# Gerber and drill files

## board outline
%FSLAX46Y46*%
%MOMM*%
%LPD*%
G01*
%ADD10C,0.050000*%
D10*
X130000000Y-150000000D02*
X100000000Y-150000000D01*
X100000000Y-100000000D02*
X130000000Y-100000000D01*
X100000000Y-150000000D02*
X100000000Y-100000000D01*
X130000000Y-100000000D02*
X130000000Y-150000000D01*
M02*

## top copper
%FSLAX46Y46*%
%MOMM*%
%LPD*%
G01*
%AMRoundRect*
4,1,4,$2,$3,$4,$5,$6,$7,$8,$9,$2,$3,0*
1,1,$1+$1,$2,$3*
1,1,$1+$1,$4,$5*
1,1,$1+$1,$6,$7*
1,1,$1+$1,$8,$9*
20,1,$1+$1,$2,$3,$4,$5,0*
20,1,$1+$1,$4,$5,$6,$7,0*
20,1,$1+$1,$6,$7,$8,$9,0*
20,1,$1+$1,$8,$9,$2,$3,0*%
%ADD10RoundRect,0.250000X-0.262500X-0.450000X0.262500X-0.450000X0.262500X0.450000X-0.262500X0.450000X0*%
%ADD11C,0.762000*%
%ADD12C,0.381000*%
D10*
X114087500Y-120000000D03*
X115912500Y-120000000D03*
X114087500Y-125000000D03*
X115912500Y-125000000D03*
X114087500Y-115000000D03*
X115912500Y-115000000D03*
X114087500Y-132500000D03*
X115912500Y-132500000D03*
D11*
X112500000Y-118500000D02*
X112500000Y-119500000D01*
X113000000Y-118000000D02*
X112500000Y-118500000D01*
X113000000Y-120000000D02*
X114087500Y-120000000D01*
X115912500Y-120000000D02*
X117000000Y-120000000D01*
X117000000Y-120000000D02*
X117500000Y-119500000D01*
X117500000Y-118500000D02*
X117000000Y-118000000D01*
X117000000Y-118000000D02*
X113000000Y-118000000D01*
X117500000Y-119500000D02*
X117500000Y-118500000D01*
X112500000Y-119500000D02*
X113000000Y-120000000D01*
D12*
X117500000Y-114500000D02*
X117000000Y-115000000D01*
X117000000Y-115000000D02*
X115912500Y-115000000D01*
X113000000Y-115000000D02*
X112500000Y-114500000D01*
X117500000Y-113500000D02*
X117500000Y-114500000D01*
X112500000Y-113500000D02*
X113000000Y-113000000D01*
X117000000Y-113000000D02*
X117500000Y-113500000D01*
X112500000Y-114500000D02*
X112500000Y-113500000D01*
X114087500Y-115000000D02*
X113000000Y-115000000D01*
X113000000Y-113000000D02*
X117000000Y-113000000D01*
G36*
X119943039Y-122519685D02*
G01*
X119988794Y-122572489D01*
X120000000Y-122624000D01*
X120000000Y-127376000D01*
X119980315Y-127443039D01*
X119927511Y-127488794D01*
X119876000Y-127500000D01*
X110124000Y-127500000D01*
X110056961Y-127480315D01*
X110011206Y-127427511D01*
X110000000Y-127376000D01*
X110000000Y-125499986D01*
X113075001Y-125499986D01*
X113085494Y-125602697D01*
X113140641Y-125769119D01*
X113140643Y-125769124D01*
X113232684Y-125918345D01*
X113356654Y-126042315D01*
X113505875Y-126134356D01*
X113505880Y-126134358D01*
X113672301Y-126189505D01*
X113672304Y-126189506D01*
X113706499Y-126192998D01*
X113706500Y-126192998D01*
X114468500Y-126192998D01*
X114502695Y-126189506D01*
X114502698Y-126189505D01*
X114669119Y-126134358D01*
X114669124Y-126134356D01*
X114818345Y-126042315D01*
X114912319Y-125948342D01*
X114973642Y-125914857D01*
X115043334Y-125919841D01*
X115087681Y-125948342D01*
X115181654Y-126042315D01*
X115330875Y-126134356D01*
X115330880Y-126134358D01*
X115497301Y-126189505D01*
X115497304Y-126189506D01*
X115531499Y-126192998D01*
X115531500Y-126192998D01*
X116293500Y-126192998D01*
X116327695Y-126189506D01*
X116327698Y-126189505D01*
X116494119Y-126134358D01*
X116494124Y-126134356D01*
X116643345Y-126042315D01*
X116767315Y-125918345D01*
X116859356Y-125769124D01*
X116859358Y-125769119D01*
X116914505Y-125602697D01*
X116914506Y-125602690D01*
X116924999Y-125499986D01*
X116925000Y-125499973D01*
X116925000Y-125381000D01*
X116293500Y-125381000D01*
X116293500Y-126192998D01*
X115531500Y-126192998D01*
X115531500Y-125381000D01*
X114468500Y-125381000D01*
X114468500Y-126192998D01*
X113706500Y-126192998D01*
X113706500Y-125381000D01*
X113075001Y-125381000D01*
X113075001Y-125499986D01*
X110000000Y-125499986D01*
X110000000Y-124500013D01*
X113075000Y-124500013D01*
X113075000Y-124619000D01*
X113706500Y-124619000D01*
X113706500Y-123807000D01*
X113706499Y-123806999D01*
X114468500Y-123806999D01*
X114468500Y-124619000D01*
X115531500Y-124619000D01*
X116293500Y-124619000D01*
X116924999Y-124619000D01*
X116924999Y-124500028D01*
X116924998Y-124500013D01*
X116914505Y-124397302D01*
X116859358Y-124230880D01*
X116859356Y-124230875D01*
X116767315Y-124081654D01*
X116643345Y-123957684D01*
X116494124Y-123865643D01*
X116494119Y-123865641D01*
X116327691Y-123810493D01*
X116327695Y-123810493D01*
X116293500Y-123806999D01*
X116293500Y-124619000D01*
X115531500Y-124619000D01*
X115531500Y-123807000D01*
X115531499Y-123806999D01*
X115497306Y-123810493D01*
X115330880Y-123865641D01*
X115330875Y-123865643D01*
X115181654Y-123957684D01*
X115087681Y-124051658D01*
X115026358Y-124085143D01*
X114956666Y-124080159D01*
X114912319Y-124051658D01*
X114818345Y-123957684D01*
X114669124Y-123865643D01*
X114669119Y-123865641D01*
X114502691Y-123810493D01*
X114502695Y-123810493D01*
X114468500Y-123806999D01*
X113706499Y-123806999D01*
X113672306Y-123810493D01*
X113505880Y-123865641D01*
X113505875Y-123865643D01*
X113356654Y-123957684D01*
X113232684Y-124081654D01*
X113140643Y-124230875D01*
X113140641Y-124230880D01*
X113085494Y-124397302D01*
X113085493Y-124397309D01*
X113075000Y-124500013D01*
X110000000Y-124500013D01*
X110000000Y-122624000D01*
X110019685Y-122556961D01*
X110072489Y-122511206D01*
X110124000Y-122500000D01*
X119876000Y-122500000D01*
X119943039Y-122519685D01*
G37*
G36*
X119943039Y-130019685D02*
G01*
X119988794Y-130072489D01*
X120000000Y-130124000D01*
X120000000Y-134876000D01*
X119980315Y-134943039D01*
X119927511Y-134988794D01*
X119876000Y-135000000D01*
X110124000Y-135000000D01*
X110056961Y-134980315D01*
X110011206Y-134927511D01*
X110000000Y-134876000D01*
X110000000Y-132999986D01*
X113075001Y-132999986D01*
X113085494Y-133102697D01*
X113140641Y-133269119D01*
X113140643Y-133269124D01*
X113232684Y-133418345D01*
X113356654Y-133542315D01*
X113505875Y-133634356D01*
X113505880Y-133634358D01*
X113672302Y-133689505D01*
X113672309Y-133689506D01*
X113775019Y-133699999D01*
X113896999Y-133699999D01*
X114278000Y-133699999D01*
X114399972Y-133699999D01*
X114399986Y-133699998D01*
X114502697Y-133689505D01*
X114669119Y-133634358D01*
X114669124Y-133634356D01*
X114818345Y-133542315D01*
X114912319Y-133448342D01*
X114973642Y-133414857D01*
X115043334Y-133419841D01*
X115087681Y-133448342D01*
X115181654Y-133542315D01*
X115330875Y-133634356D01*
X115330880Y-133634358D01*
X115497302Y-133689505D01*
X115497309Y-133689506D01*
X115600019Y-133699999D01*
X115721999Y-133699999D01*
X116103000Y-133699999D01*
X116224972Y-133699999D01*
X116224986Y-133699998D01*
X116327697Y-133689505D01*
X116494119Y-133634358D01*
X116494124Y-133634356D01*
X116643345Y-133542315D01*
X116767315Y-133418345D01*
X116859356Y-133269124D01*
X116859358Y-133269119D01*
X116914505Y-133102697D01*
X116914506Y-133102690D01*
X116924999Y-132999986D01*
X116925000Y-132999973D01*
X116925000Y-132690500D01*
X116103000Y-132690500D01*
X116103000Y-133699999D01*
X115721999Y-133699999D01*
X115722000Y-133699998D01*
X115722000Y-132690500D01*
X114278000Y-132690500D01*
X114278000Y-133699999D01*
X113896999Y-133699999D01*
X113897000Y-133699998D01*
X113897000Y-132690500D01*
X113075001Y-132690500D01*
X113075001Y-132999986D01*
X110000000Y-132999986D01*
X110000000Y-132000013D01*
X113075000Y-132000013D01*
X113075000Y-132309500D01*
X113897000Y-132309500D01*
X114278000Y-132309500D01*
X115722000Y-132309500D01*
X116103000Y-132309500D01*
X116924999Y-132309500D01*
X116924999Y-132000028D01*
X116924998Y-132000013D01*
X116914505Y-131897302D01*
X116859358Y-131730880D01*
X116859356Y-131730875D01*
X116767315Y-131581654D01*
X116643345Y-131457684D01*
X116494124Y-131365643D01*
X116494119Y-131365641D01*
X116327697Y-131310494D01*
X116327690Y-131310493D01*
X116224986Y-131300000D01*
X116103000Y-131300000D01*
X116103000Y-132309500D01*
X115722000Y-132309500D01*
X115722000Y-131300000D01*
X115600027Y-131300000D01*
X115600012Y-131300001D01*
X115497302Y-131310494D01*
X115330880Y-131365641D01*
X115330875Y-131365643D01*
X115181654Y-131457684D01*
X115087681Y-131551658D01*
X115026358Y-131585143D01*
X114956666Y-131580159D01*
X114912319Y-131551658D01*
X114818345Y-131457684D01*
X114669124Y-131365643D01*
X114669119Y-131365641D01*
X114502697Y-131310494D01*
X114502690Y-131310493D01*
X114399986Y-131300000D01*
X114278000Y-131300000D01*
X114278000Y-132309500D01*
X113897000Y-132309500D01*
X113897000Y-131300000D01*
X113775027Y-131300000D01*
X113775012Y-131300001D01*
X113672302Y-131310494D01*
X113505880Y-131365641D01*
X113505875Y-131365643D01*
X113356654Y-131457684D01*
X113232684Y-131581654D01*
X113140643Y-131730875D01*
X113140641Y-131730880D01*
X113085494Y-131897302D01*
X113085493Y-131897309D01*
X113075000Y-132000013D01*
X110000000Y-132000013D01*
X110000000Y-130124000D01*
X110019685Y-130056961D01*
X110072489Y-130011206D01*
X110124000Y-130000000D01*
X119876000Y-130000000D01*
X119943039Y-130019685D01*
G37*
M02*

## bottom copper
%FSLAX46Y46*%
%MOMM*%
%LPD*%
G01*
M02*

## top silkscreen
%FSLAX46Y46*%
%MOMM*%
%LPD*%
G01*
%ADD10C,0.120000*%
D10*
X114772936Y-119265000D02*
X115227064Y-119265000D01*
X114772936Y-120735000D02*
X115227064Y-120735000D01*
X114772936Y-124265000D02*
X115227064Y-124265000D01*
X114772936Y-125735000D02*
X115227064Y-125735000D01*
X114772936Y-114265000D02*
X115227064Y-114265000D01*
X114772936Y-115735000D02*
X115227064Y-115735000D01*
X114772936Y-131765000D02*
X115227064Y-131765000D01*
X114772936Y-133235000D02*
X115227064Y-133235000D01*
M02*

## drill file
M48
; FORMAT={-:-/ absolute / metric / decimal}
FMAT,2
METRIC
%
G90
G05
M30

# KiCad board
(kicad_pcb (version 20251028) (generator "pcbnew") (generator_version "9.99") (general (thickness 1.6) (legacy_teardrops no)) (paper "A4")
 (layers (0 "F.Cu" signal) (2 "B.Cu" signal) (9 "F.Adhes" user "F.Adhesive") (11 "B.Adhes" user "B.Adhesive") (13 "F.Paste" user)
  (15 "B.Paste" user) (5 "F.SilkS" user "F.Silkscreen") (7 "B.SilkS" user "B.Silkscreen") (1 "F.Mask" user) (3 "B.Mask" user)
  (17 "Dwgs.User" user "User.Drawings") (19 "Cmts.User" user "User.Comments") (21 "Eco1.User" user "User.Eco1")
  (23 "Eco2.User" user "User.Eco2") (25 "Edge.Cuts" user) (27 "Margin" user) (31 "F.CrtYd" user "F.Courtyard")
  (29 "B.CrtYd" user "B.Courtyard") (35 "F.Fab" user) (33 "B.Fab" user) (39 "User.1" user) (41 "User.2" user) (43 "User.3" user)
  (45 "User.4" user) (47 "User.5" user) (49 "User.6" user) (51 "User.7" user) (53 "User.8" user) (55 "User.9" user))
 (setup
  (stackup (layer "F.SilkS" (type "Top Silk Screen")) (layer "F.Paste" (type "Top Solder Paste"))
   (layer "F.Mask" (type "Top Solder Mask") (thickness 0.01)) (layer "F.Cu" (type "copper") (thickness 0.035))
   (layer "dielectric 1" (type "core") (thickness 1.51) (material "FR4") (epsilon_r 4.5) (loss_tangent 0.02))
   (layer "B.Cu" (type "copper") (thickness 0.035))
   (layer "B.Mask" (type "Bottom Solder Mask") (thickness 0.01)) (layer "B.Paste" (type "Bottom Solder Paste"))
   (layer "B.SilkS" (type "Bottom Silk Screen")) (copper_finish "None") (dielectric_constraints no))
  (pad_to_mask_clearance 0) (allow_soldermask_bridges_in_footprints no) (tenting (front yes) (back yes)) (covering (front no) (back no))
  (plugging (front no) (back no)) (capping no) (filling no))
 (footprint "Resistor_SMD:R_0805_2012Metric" (layer "F.Cu") (at 115 120)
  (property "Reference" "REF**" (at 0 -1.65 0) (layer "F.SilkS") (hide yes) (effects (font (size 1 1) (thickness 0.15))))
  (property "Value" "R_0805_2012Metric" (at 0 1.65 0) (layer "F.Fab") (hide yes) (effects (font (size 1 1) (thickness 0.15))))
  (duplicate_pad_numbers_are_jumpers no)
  (fp_line (start -0.227064 -0.735) (end 0.227064 -0.735) (stroke (width 0.12) (type solid)) (layer "F.SilkS"))
  (fp_line (start -0.227064 0.735) (end 0.227064 0.735) (stroke (width 0.12) (type solid)) (layer "F.SilkS"))
  (pad "1" smd roundrect (at -0.9125 0) (size 1.025 1.4) (layers "F.Cu" "F.Mask" "F.Paste") (roundrect_rratio 0.243902) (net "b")
   (tenting (front none) (back none)))
  (pad "2" smd roundrect (at 0.9125 0) (size 1.025 1.4) (layers "F.Cu" "F.Mask" "F.Paste") (roundrect_rratio 0.243902) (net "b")
   (tenting (front none) (back none))))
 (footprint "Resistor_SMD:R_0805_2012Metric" (layer "F.Cu") (at 115 125)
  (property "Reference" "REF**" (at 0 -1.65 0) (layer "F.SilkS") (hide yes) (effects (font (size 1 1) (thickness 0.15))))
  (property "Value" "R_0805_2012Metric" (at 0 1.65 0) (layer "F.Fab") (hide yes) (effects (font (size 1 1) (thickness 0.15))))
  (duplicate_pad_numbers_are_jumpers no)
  (fp_line (start -0.227064 -0.735) (end 0.227064 -0.735) (stroke (width 0.12) (type solid)) (layer "F.SilkS"))
  (fp_line (start -0.227064 0.735) (end 0.227064 0.735) (stroke (width 0.12) (type solid)) (layer "F.SilkS"))
  (pad "1" smd roundrect (at -0.9125 0) (size 1.025 1.4) (layers "F.Cu" "F.Mask" "F.Paste") (roundrect_rratio 0.243902) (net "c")
   (tenting (front none) (back none)))
  (pad "2" smd roundrect (at 0.9125 0) (size 1.025 1.4) (layers "F.Cu" "F.Mask" "F.Paste") (roundrect_rratio 0.243902) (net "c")
   (tenting (front none) (back none))))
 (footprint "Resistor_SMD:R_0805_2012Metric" (layer "F.Cu") (at 115 115)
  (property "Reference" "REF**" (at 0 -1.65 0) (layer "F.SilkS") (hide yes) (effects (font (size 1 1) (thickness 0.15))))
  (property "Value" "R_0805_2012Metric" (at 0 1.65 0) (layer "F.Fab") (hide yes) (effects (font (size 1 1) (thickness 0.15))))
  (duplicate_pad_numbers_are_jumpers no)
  (fp_line (start -0.227064 -0.735) (end 0.227064 -0.735) (stroke (width 0.12) (type solid)) (layer "F.SilkS"))
  (fp_line (start -0.227064 0.735) (end 0.227064 0.735) (stroke (width 0.12) (type solid)) (layer "F.SilkS"))
  (pad "1" smd roundrect (at -0.9125 0) (size 1.025 1.4) (layers "F.Cu" "F.Mask" "F.Paste") (roundrect_rratio 0.243902) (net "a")
   (tenting (front none) (back none)))
  (pad "2" smd roundrect (at 0.9125 0) (size 1.025 1.4) (layers "F.Cu" "F.Mask" "F.Paste") (roundrect_rratio 0.243902) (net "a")
   (tenting (front none) (back none))))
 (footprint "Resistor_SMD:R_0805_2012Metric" (layer "F.Cu") (at 115 132.5)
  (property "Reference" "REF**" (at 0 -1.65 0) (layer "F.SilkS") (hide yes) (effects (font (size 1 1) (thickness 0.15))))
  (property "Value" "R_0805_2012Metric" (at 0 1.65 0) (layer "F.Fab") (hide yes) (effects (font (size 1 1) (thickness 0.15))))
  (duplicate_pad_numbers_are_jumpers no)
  (fp_line (start -0.227064 -0.735) (end 0.227064 -0.735) (stroke (width 0.12) (type solid)) (layer "F.SilkS"))
  (fp_line (start -0.227064 0.735) (end 0.227064 0.735) (stroke (width 0.12) (type solid)) (layer "F.SilkS"))
  (pad "1" smd roundrect (at -0.9125 0) (size 1.025 1.4) (layers "F.Cu" "F.Mask" "F.Paste") (roundrect_rratio 0.243902) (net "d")
   (tenting (front none) (back none)))
  (pad "2" smd roundrect (at 0.9125 0) (size 1.025 1.4) (layers "F.Cu" "F.Mask" "F.Paste") (roundrect_rratio 0.243902) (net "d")
   (tenting (front none) (back none))))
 (gr_line (start 130 150) (end 100 150) (stroke (width 0.05) (type default)) (layer "Edge.Cuts"))
 (gr_line (start 100 100) (end 130 100) (stroke (width 0.05) (type default)) (layer "Edge.Cuts"))
 (gr_line (start 100 150) (end 100 100) (stroke (width 0.05) (type default)) (layer "Edge.Cuts"))
 (gr_line (start 130 100) (end 130 150) (stroke (width 0.05) (type default)) (layer "Edge.Cuts"))
 (segment (start 112.5 118.5) (end 112.5 119.5) (width 0.762) (layer "F.Cu") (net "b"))
 (segment (start 113 118) (end 112.5 118.5) (width 0.762) (layer "F.Cu") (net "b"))
 (segment (start 113 120) (end 114.0875 120) (width 0.762) (layer "F.Cu") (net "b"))
 (segment (start 115.9125 120) (end 117 120) (width 0.762) (layer "F.Cu") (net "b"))
 (segment (start 117 120) (end 117.5 119.5) (width 0.762) (layer "F.Cu") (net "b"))
 (segment (start 117.5 118.5) (end 117 118) (width 0.762) (layer "F.Cu") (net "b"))
 (segment (start 117 118) (end 113 118) (width 0.762) (layer "F.Cu") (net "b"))
 (segment (start 117.5 119.5) (end 117.5 118.5) (width 0.762) (layer "F.Cu") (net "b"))
 (segment (start 112.5 119.5) (end 113 120) (width 0.762) (layer "F.Cu") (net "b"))
 (segment (start 117.5 114.5) (end 117 115) (width 0.381) (layer "F.Cu") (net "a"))
 (segment (start 117 115) (end 115.9125 115) (width 0.381) (layer "F.Cu") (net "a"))
 (segment (start 113 115) (end 112.5 114.5) (width 0.381) (layer "F.Cu") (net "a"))
 (segment (start 117.5 113.5) (end 117.5 114.5) (width 0.381) (layer "F.Cu") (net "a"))
 (segment (start 112.5 113.5) (end 113 113) (width 0.381) (layer "F.Cu") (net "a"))
 (segment (start 117 113) (end 117.5 113.5) (width 0.381) (layer "F.Cu") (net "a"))
 (segment (start 112.5 114.5) (end 112.5 113.5) (width 0.381) (layer "F.Cu") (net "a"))
 (segment (start 114.0875 115) (end 113 115) (width 0.381) (layer "F.Cu") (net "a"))
 (segment (start 113 113) (end 117 113) (width 0.381) (layer "F.Cu") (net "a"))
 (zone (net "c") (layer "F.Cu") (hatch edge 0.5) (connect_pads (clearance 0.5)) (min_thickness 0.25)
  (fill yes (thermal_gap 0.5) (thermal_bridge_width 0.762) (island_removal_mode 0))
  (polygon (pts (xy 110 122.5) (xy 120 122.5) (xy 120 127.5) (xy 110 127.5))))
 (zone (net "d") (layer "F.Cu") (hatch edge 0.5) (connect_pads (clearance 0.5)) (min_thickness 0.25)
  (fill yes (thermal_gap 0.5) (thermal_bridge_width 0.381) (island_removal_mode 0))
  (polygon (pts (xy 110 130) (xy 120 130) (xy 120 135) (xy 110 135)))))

